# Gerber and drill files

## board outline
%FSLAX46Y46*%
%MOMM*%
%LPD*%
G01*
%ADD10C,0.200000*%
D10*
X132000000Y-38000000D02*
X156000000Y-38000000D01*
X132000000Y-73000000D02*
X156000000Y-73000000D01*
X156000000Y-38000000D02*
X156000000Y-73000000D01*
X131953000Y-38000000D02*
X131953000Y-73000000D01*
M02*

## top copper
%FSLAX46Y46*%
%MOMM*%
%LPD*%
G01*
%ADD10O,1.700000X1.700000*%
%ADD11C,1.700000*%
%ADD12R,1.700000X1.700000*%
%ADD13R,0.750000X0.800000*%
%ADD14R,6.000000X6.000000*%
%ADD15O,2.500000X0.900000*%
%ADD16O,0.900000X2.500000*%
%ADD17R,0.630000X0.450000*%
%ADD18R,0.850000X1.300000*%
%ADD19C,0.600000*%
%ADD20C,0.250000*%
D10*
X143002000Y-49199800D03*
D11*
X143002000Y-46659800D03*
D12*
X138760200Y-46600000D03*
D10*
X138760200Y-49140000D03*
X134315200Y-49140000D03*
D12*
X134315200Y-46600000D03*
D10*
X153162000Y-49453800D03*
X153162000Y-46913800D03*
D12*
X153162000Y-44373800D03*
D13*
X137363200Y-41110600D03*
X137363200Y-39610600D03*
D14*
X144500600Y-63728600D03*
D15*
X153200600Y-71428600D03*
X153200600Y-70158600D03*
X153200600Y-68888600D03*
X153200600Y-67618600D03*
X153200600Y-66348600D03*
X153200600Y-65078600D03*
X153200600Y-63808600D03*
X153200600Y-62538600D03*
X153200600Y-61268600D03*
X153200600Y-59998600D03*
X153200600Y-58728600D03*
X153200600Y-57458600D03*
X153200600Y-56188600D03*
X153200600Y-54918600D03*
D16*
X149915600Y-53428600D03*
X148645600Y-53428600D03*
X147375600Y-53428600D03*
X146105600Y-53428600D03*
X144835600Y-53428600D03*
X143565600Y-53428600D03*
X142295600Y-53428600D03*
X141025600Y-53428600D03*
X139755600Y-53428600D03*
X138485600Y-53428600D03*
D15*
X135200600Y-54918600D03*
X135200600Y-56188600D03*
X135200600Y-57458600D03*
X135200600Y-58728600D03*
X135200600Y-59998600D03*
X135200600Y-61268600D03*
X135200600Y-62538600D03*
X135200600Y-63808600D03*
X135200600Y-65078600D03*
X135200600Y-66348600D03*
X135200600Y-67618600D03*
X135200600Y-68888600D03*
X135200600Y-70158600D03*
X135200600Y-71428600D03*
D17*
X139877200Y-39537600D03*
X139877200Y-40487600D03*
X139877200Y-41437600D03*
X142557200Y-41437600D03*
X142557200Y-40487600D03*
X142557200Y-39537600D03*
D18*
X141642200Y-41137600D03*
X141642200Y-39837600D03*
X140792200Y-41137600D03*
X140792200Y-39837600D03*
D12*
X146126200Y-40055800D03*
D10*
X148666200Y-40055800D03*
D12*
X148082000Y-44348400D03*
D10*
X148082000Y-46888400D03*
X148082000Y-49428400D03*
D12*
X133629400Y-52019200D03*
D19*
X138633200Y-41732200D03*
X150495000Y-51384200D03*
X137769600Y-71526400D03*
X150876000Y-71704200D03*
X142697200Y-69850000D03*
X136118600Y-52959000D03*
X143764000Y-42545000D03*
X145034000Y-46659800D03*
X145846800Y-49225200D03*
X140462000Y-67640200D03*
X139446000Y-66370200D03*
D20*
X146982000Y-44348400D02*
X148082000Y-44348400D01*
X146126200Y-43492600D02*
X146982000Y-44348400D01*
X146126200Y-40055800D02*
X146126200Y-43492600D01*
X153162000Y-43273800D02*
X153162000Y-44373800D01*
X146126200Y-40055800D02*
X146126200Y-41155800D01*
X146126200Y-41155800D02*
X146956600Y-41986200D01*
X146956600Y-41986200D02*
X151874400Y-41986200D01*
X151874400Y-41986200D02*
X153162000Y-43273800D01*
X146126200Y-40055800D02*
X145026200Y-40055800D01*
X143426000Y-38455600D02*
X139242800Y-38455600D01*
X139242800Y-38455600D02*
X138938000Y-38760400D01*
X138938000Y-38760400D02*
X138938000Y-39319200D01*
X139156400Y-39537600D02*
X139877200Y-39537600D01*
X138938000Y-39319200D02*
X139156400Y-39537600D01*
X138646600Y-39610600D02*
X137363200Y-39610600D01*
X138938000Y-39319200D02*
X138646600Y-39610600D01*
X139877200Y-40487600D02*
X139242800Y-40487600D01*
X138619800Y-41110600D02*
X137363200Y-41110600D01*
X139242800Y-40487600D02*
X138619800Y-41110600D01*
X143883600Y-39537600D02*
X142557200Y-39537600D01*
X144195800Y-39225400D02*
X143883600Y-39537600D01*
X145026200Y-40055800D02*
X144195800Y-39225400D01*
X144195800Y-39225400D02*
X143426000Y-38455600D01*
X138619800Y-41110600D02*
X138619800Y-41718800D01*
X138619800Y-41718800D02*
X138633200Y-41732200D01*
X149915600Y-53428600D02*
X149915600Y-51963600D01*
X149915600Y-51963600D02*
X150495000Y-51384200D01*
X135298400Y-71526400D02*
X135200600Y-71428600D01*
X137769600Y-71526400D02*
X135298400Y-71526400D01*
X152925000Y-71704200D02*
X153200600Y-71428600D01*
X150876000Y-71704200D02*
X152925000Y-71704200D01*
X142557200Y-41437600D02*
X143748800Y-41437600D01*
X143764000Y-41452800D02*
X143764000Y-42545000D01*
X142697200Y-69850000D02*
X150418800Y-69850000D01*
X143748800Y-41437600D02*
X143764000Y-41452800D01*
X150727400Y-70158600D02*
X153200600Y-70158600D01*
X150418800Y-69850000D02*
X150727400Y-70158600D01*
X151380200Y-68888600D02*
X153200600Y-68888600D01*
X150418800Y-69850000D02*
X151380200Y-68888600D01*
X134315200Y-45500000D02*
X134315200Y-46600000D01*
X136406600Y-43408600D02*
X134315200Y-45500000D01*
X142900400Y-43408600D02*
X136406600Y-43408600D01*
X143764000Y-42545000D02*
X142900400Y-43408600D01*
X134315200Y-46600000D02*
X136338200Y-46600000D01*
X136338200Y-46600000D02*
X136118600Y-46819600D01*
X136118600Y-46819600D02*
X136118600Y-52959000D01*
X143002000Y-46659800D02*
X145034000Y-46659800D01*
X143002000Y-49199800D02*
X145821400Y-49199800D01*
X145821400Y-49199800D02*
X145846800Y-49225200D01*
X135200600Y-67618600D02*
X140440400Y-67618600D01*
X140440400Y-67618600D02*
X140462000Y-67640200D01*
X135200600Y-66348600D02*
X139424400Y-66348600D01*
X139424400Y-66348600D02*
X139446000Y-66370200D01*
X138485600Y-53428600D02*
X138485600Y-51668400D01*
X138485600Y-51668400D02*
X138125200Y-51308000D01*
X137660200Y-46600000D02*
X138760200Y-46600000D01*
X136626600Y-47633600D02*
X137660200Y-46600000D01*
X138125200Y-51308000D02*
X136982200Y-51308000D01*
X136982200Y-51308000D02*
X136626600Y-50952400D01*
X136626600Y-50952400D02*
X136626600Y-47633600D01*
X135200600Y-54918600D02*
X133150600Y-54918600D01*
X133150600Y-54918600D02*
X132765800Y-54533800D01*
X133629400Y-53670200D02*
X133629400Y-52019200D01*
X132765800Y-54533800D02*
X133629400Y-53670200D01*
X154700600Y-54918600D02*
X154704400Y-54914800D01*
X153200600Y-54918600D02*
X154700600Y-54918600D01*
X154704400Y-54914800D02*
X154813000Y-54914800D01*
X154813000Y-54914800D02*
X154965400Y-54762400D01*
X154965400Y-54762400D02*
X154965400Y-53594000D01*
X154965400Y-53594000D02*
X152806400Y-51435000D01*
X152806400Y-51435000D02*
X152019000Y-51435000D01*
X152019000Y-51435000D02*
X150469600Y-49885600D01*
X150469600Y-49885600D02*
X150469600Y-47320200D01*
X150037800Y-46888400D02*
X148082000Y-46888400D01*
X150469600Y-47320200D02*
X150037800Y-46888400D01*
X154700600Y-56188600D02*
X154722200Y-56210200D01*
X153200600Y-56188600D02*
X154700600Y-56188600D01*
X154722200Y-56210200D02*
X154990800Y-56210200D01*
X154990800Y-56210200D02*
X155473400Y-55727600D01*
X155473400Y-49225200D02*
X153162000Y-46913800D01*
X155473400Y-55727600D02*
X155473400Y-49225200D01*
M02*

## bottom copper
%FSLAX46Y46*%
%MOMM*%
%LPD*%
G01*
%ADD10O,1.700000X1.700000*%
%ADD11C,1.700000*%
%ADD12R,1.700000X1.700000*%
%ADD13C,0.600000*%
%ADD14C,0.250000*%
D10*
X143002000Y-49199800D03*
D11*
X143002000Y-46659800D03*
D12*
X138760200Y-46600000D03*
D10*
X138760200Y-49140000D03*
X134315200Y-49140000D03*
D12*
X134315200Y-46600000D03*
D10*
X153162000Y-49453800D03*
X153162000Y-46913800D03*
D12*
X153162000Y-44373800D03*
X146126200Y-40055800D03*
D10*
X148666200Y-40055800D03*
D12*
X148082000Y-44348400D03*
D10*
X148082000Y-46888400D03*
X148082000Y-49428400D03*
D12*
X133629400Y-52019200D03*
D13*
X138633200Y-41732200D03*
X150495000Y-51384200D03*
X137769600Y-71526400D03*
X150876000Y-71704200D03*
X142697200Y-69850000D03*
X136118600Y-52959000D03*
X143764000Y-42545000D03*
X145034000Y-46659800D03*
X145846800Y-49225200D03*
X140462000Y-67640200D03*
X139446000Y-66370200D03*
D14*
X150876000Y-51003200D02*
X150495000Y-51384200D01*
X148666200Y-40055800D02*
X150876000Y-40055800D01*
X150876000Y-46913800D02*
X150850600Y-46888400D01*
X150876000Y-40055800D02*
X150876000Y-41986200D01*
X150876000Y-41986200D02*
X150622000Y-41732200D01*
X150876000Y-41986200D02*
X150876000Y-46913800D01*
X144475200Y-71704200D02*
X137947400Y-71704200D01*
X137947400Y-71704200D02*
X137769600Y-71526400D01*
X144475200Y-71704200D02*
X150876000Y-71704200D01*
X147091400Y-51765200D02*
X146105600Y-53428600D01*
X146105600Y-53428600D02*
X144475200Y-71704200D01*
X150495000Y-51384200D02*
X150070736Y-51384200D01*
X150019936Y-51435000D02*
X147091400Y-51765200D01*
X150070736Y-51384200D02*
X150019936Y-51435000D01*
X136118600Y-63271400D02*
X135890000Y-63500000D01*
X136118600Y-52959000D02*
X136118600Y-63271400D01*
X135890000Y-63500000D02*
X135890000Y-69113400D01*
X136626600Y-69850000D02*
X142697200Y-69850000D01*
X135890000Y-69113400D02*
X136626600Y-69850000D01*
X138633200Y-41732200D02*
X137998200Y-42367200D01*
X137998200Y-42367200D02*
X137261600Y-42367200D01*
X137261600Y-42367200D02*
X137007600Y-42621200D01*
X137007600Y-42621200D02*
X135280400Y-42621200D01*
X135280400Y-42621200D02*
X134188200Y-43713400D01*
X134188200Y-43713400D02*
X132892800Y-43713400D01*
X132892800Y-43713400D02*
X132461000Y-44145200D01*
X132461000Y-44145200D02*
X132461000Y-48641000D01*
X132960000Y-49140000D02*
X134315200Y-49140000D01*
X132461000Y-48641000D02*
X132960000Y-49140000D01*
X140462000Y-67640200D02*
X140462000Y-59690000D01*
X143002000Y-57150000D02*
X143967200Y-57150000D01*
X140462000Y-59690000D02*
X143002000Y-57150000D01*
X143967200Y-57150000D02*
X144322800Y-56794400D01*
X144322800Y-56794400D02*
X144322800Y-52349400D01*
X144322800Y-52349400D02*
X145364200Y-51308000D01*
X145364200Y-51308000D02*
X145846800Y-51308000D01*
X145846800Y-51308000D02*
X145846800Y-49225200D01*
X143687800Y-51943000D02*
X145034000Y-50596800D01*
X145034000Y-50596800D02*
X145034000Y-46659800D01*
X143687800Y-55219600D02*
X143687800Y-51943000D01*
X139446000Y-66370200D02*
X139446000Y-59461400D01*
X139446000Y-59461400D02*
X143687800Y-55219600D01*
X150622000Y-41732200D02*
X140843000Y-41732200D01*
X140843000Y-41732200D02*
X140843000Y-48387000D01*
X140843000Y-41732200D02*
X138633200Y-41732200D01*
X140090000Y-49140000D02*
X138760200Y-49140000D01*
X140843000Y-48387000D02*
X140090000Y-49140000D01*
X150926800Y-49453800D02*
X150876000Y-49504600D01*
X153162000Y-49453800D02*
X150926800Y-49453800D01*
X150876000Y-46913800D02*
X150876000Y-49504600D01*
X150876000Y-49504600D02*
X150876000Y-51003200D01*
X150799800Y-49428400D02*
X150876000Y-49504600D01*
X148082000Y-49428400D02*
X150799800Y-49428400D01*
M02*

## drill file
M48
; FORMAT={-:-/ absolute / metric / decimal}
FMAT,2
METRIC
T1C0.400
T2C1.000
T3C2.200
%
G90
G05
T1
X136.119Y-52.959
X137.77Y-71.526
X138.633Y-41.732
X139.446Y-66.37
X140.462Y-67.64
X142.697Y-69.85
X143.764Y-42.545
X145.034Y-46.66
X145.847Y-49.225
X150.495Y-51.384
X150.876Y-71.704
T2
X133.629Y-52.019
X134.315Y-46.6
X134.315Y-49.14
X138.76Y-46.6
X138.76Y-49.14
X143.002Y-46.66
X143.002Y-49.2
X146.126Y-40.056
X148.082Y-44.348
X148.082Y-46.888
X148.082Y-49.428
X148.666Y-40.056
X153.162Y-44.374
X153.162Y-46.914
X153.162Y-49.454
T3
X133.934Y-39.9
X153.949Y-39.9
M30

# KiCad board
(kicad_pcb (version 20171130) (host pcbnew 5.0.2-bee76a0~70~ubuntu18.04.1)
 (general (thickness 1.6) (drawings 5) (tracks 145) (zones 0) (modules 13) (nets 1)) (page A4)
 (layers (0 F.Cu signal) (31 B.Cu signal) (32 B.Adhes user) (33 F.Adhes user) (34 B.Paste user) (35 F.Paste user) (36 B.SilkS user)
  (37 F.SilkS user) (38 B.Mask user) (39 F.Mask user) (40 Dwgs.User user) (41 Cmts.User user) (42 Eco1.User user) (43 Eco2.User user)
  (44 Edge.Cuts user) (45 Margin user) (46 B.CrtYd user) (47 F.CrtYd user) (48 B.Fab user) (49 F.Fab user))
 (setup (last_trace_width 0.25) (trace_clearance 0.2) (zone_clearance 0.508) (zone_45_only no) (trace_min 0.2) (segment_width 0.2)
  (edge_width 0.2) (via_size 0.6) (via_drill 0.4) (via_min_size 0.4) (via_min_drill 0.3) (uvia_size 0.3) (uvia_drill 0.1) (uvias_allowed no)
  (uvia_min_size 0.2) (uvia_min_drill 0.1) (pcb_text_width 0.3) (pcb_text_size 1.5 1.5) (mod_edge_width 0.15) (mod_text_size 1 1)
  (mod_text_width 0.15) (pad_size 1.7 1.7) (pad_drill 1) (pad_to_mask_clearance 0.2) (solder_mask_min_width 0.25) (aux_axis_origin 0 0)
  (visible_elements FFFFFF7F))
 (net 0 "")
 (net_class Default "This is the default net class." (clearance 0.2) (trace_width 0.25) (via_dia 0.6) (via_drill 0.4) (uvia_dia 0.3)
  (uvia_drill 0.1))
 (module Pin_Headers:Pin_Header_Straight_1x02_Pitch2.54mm (layer F.Cu) (at 143.002 46.6598)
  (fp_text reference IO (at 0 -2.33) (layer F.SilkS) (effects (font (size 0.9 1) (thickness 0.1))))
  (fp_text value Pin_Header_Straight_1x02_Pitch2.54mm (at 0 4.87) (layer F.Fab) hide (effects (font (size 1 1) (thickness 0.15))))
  (pad 2 thru_hole oval (at 0 2.54) (size 1.7 1.7) (drill 1) (layers *.Cu *.Mask))
  (pad 1 thru_hole circle (at 0 0) (size 1.7 1.7) (drill 1) (layers *.Cu *.Mask)))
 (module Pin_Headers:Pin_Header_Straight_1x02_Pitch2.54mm (layer F.Cu) (at 138.7602 46.6)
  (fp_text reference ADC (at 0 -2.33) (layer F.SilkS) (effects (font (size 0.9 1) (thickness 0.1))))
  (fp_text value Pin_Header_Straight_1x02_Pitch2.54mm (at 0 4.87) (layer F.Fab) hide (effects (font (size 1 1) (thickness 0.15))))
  (pad 1 thru_hole rect (at 0 0) (size 1.7 1.7) (drill 1) (layers *.Cu *.Mask))
  (pad 2 thru_hole oval (at 0 2.54) (size 1.7 1.7) (drill 1) (layers *.Cu *.Mask)))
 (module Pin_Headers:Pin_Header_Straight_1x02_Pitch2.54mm (layer F.Cu) (at 134.3152 46.6)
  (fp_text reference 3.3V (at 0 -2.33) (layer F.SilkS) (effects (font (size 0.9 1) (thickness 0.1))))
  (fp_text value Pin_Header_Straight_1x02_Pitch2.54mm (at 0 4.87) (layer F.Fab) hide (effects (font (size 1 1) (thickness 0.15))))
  (pad 2 thru_hole oval (at 0 2.54) (size 1.7 1.7) (drill 1) (layers *.Cu *.Mask))
  (pad 1 thru_hole rect (at 0 0) (size 1.7 1.7) (drill 1) (layers *.Cu *.Mask)))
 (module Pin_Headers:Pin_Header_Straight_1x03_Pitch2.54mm (layer F.Cu) (at 153.162 44.3738)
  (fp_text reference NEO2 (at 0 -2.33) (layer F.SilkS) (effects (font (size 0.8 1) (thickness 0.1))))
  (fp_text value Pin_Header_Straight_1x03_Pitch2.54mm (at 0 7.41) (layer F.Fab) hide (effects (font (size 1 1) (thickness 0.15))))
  (pad 3 thru_hole oval (at 0 5.08) (size 1.7 1.7) (drill 1) (layers *.Cu *.Mask))
  (pad 2 thru_hole oval (at 0 2.54) (size 1.7 1.7) (drill 1) (layers *.Cu *.Mask))
  (pad 1 thru_hole rect (at 0 0) (size 1.7 1.7) (drill 1) (layers *.Cu *.Mask)))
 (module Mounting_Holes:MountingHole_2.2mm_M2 (layer F.Cu) (at 133.9342 39.9)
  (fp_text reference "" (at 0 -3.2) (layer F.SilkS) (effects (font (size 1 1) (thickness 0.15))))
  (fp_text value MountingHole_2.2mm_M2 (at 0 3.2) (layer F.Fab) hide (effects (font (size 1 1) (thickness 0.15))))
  (pad 1 np_thru_hole circle (at 0 0) (size 2.2 2.2) (drill 2.2) (layers *.Cu *.Mask F.SilkS)))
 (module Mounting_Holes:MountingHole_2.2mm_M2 (layer F.Cu) (at 153.9494 39.9)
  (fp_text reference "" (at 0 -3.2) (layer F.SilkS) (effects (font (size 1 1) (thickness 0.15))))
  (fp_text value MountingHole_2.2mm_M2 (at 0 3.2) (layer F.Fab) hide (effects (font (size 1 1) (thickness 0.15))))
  (pad 1 np_thru_hole circle (at 0 0) (size 2.2 2.2) (drill 2.2) (layers *.Cu *.Mask F.SilkS)))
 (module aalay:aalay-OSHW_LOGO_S (layer B.Cu) (at 139.9794 40.4876)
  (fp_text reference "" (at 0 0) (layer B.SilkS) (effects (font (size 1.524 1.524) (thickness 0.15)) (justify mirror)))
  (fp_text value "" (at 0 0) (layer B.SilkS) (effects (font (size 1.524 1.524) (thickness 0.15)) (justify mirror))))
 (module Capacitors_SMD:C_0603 (layer F.Cu) (at 137.3632 40.3606 90)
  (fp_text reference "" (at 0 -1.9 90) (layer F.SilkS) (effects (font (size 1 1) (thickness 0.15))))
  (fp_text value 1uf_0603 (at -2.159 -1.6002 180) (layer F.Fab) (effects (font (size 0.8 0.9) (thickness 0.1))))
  (pad 1 smd rect (at -0.75 0 90) (size 0.8 0.75) (layers F.Cu F.Paste F.Mask))
  (pad 2 smd rect (at 0.75 0 90) (size 0.8 0.75) (layers F.Cu F.Paste F.Mask)))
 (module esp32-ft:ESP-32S (layer F.Cu) (at 144.148034 61.911262 180)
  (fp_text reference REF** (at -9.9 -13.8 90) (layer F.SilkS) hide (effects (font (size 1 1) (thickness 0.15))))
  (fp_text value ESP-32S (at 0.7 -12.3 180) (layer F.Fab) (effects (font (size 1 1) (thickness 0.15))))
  (pad 39 smd rect (at -0.352566 -1.817338) (size 6 6) (layers F.Cu F.Paste F.Mask))
  (pad 1 smd oval (at -9.052566 -9.517338) (size 2.5 0.9) (layers F.Cu F.Paste F.Mask))
  (pad 2 smd oval (at -9.052566 -8.247338) (size 2.5 0.9) (layers F.Cu F.Paste F.Mask))
  (pad 3 smd oval (at -9.052566 -6.977338) (size 2.5 0.9) (layers F.Cu F.Paste F.Mask))
  (pad 4 smd oval (at -9.052566 -5.707338) (size 2.5 0.9) (layers F.Cu F.Paste F.Mask))
  (pad 5 smd oval (at -9.052566 -4.437338) (size 2.5 0.9) (layers F.Cu F.Paste F.Mask))
  (pad 6 smd oval (at -9.052566 -3.167338) (size 2.5 0.9) (layers F.Cu F.Paste F.Mask))
  (pad 7 smd oval (at -9.052566 -1.897338) (size 2.5 0.9) (layers F.Cu F.Paste F.Mask))
  (pad 8 smd oval (at -9.052566 -0.627338) (size 2.5 0.9) (layers F.Cu F.Paste F.Mask))
  (pad 9 smd oval (at -9.052566 0.642662) (size 2.5 0.9) (layers F.Cu F.Paste F.Mask))
  (pad 10 smd oval (at -9.052566 1.912662) (size 2.5 0.9) (layers F.Cu F.Paste F.Mask))
  (pad 11 smd oval (at -9.052566 3.182662) (size 2.5 0.9) (layers F.Cu F.Paste F.Mask))
  (pad 12 smd oval (at -9.052566 4.452662) (size 2.5 0.9) (layers F.Cu F.Paste F.Mask))
  (pad 13 smd oval (at -9.052566 5.722662) (size 2.5 0.9) (layers F.Cu F.Paste F.Mask))
  (pad 14 smd oval (at -9.052566 6.992662) (size 2.5 0.9) (layers F.Cu F.Paste F.Mask))
  (pad 15 smd oval (at -5.767566 8.482662) (size 0.9 2.5) (layers F.Cu F.Paste F.Mask))
  (pad 16 smd oval (at -4.497566 8.482662) (size 0.9 2.5) (layers F.Cu F.Paste F.Mask))
  (pad 17 smd oval (at -3.227566 8.482662) (size 0.9 2.5) (layers F.Cu F.Paste F.Mask))
  (pad 18 smd oval (at -1.957566 8.482662) (size 0.9 2.5) (layers F.Cu F.Paste F.Mask))
  (pad 19 smd oval (at -0.687566 8.482662) (size 0.9 2.5) (layers F.Cu F.Paste F.Mask))
  (pad 20 smd oval (at 0.582434 8.482662) (size 0.9 2.5) (layers F.Cu F.Paste F.Mask))
  (pad 21 smd oval (at 1.852434 8.482662) (size 0.9 2.5) (layers F.Cu F.Paste F.Mask))
  (pad 22 smd oval (at 3.122434 8.482662) (size 0.9 2.5) (layers F.Cu F.Paste F.Mask))
  (pad 23 smd oval (at 4.392434 8.482662) (size 0.9 2.5) (layers F.Cu F.Paste F.Mask))
  (pad 24 smd oval (at 5.662434 8.482662) (size 0.9 2.5) (layers F.Cu F.Paste F.Mask))
  (pad 25 smd oval (at 8.947434 6.992662) (size 2.5 0.9) (layers F.Cu F.Paste F.Mask))
  (pad 26 smd oval (at 8.947434 5.722662) (size 2.5 0.9) (layers F.Cu F.Paste F.Mask))
  (pad 27 smd oval (at 8.947434 4.452662) (size 2.5 0.9) (layers F.Cu F.Paste F.Mask))
  (pad 28 smd oval (at 8.947434 3.182662) (size 2.5 0.9) (layers F.Cu F.Paste F.Mask))
  (pad 29 smd oval (at 8.947434 1.912662) (size 2.5 0.9) (layers F.Cu F.Paste F.Mask))
  (pad 30 smd oval (at 8.947434 0.642662) (size 2.5 0.9) (layers F.Cu F.Paste F.Mask))
  (pad 31 smd oval (at 8.947434 -0.627338) (size 2.5 0.9) (layers F.Cu F.Paste F.Mask))
  (pad 32 smd oval (at 8.947434 -1.897338) (size 2.5 0.9) (layers F.Cu F.Paste F.Mask))
  (pad 33 smd oval (at 8.947434 -3.167338) (size 2.5 0.9) (layers F.Cu F.Paste F.Mask))
  (pad 34 smd oval (at 8.947434 -4.437338) (size 2.5 0.9) (layers F.Cu F.Paste F.Mask))
  (pad 35 smd oval (at 8.947434 -5.707338) (size 2.5 0.9) (layers F.Cu F.Paste F.Mask))
  (pad 36 smd oval (at 8.947434 -6.977338) (size 2.5 0.9) (layers F.Cu F.Paste F.Mask))
  (pad 37 smd oval (at 8.947434 -8.247338) (size 2.5 0.9) (layers F.Cu F.Paste F.Mask))
  (pad 38 smd oval (at 8.947434 -9.517338) (size 2.5 0.9) (layers F.Cu F.Paste F.Mask)))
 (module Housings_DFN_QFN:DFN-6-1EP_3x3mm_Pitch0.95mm (layer F.Cu) (at 141.2172 40.4876)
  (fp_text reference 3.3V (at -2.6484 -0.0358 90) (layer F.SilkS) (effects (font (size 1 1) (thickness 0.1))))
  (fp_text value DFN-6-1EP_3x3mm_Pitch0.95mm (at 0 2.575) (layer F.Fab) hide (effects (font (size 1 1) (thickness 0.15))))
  (pad 1 smd rect (at -1.34 -0.95) (size 0.63 0.45) (layers F.Cu F.Paste F.Mask))
  (pad 2 smd rect (at -1.34 0) (size 0.63 0.45) (layers F.Cu F.Paste F.Mask))
  (pad 3 smd rect (at -1.34 0.95) (size 0.63 0.45) (layers F.Cu F.Paste F.Mask))
  (pad 4 smd rect (at 1.34 0.95) (size 0.63 0.45) (layers F.Cu F.Paste F.Mask))
  (pad 5 smd rect (at 1.34 0) (size 0.63 0.45) (layers F.Cu F.Paste F.Mask))
  (pad 6 smd rect (at 1.34 -0.95) (size 0.63 0.45) (layers F.Cu F.Paste F.Mask))
  (pad 7 smd rect (at 0.425 0.65) (size 0.85 1.3) (layers F.Cu F.Paste F.Mask) (solder_paste_margin_ratio -0.2))
  (pad 7 smd rect (at 0.425 -0.65) (size 0.85 1.3) (layers F.Cu F.Paste F.Mask) (solder_paste_margin_ratio -0.2))
  (pad 7 smd rect (at -0.425 0.65) (size 0.85 1.3) (layers F.Cu F.Paste F.Mask) (solder_paste_margin_ratio -0.2))
  (pad 7 smd rect (at -0.425 -0.65) (size 0.85 1.3) (layers F.Cu F.Paste F.Mask) (solder_paste_margin_ratio -0.2)))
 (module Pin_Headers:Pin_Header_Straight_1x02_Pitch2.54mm (layer F.Cu) (at 146.1262 40.0558 90)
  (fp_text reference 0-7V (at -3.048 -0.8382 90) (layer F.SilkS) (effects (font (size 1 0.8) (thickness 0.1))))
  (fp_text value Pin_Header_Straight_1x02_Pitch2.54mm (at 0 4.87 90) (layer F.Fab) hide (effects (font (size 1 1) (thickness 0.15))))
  (pad 1 thru_hole rect (at 0 0 90) (size 1.7 1.7) (drill 1) (layers *.Cu *.Mask))
  (pad 2 thru_hole oval (at 0 2.54 90) (size 1.7 1.7) (drill 1) (layers *.Cu *.Mask)))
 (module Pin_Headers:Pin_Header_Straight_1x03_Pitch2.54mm (layer F.Cu) (at 148.082 44.3484)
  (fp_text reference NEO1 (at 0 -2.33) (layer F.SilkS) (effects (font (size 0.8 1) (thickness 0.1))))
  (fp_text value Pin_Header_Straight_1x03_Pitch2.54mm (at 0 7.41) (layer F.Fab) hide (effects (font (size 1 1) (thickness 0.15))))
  (pad 1 thru_hole rect (at 0 0) (size 1.7 1.7) (drill 1) (layers *.Cu *.Mask))
  (pad 2 thru_hole oval (at 0 2.54) (size 1.7 1.7) (drill 1) (layers *.Cu *.Mask))
  (pad 3 thru_hole oval (at 0 5.08) (size 1.7 1.7) (drill 1) (layers *.Cu *.Mask)))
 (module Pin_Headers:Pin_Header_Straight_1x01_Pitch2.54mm (layer F.Cu) (at 133.6294 52.0192)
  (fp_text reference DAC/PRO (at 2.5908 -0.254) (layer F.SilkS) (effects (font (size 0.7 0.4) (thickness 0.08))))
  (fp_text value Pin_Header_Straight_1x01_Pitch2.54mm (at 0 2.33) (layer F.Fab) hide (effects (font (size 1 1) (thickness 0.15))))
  (pad 1 thru_hole rect (at 0 0) (size 1.7 1.7) (drill 1) (layers *.Cu *.Mask)))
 (gr_line (start 132 38) (end 156 38) (angle 90) (layer Edge.Cuts) (width 0.2))
 (gr_line (start 132 73) (end 156 73) (angle 90) (layer Edge.Cuts) (width 0.2))
 (gr_line (start 156 38) (end 156 73) (angle 90) (layer Edge.Cuts) (width 0.2))
 (gr_line (start 131.953 38) (end 131.953 73) (angle 90) (layer Edge.Cuts) (width 0.2))
 (segment (start 146.982 44.3484) (end 148.082 44.3484) (width 0.25) (layer F.Cu) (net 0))
 (segment (start 146.1262 43.4926) (end 146.982 44.3484) (width 0.25) (layer F.Cu) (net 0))
 (segment (start 146.1262 40.0558) (end 146.1262 43.4926) (width 0.25) (layer F.Cu) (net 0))
 (segment (start 153.162 43.2738) (end 153.162 44.3738) (width 0.25) (layer F.Cu) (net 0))
 (segment (start 146.1262 40.0558) (end 146.1262 41.1558) (width 0.25) (layer F.Cu) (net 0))
 (segment (start 146.1262 41.1558) (end 146.9566 41.9862) (width 0.25) (layer F.Cu) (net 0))
 (segment (start 146.9566 41.9862) (end 151.8744 41.9862) (width 0.25) (layer F.Cu) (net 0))
 (segment (start 151.8744 41.9862) (end 153.162 43.2738) (width 0.25) (layer F.Cu) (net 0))
 (segment (start 146.1262 40.0558) (end 145.0262 40.0558) (width 0.25) (layer F.Cu) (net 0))
 (segment (start 143.426 38.4556) (end 139.2428 38.4556) (width 0.25) (layer F.Cu) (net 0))
 (segment (start 139.2428 38.4556) (end 138.938 38.7604) (width 0.25) (layer F.Cu) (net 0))
 (segment (start 138.938 38.7604) (end 138.938 39.3192) (width 0.25) (layer F.Cu) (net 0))
 (segment (start 139.1564 39.5376) (end 139.8772 39.5376) (width 0.25) (layer F.Cu) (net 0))
 (segment (start 138.938 39.3192) (end 139.1564 39.5376) (width 0.25) (layer F.Cu) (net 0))
 (segment (start 138.6466 39.6106) (end 137.3632 39.6106) (width 0.25) (layer F.Cu) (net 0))
 (segment (start 138.938 39.3192) (end 138.6466 39.6106) (width 0.25) (layer F.Cu) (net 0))
 (segment (start 139.8772 40.4876) (end 139.2428 40.4876) (width 0.25) (layer F.Cu) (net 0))
 (segment (start 138.6198 41.1106) (end 137.3632 41.1106) (width 0.25) (layer F.Cu) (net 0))
 (segment (start 139.2428 40.4876) (end 138.6198 41.1106) (width 0.25) (layer F.Cu) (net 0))
 (segment (start 143.8836 39.5376) (end 142.5572 39.5376) (width 0.25) (layer F.Cu) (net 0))
 (segment (start 144.1958 39.2254) (end 143.8836 39.5376) (width 0.25) (layer F.Cu) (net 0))
 (segment (start 145.0262 40.0558) (end 144.1958 39.2254) (width 0.25) (layer F.Cu) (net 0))
 (segment (start 144.1958 39.2254) (end 143.426 38.4556) (width 0.25) (layer F.Cu) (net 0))
 (segment (start 138.6198 41.1106) (end 138.6198 41.7188) (width 0.25) (layer F.Cu) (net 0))
 (via (at 138.6332 41.7322) (size 0.6) (drill 0.4) (layers F.Cu B.Cu) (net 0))
 (segment (start 138.6198 41.7188) (end 138.6332 41.7322) (width 0.25) (layer F.Cu) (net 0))
 (via (at 150.495 51.3842) (size 0.6) (drill 0.4) (layers F.Cu B.Cu) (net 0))
 (segment (start 149.9156 53.4286) (end 149.9156 51.9636) (width 0.25) (layer F.Cu) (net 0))
 (segment (start 149.9156 51.9636) (end 150.495 51.3842) (width 0.25) (layer F.Cu) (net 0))
 (segment (start 150.876 51.0032) (end 150.495 51.3842) (width 0.25) (layer B.Cu) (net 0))
 (segment (start 148.6662 40.0558) (end 150.876 40.0558) (width 0.25) (layer B.Cu) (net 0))
 (segment (start 150.876 46.9138) (end 150.8506 46.8884) (width 0.25) (layer B.Cu) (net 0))
 (segment (start 150.876 40.0558) (end 150.876 41.9862) (width 0.25) (layer B.Cu) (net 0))
 (segment (start 150.876 41.9862) (end 150.622 41.7322) (width 0.25) (layer B.Cu) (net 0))
 (segment (start 150.876 41.9862) (end 150.876 46.9138) (width 0.25) (layer B.Cu) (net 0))
 (via (at 137.7696 71.5264) (size 0.6) (drill 0.4) (layers F.Cu B.Cu) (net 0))
 (segment (start 144.4752 71.7042) (end 137.9474 71.7042) (width 0.25) (layer B.Cu) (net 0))
 (segment (start 137.9474 71.7042) (end 137.7696 71.5264) (width 0.25) (layer B.Cu) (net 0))
 (segment (start 135.2984 71.5264) (end 135.2006 71.4286) (width 0.25) (layer F.Cu) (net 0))
 (segment (start 137.7696 71.5264) (end 135.2984 71.5264) (width 0.25) (layer F.Cu) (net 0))
 (via (at 150.876 71.7042) (size 0.6) (drill 0.4) (layers F.Cu B.Cu) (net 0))
 (segment (start 144.4752 71.7042) (end 150.876 71.7042) (width 0.25) (layer B.Cu) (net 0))
 (segment (start 152.925 71.7042) (end 153.2006 71.4286) (width 0.25) (layer F.Cu) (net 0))
 (segment (start 150.876 71.7042) (end 152.925 71.7042) (width 0.25) (layer F.Cu) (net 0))
 (segment (start 142.5572 41.4376) (end 143.7488 41.4376) (width 0.25) (layer F.Cu) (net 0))
 (segment (start 143.764 41.4528) (end 143.764 42.545) (width 0.25) (layer F.Cu) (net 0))
 (segment (start 142.6972 69.85) (end 150.4188 69.85) (width 0.25) (layer F.Cu) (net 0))
 (via (at 142.6972 69.85) (size 0.6) (drill 0.4) (layers F.Cu B.Cu) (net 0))
 (segment (start 143.7488 41.4376) (end 143.764 41.4528) (width 0.25) (layer F.Cu) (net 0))
 (segment (start 150.7274 70.1586) (end 153.2006 70.1586) (width 0.25) (layer F.Cu) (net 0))
 (segment (start 150.4188 69.85) (end 150.7274 70.1586) (width 0.25) (layer F.Cu) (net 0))
 (segment (start 151.3802 68.8886) (end 153.2006 68.8886) (width 0.25) (layer F.Cu) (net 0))
 (segment (start 150.4188 69.85) (end 151.3802 68.8886) (width 0.25) (layer F.Cu) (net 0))
 (segment (start 147.0914 51.7652) (end 146.1056 53.4286) (width 0.25) (layer B.Cu) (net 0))
 (segment (start 146.1056 53.4286) (end 144.4752 71.7042) (width 0.25) (layer B.Cu) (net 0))
 (segment (start 150.495 51.3842) (end 150.070736 51.3842) (width 0.25) (layer B.Cu) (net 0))
 (segment (start 150.019936 51.435) (end 147.0914 51.7652) (width 0.25) (layer B.Cu) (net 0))
 (segment (start 150.070736 51.3842) (end 150.019936 51.435) (width 0.25) (layer B.Cu) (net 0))
 (segment (start 134.3152 45.5) (end 134.3152 46.6) (width 0.25) (layer F.Cu) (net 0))
 (segment (start 136.4066 43.4086) (end 134.3152 45.5) (width 0.25) (layer F.Cu) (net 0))
 (segment (start 142.9004 43.4086) (end 136.4066 43.4086) (width 0.25) (layer F.Cu) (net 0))
 (segment (start 143.764 42.545) (end 142.9004 43.4086) (width 0.25) (layer F.Cu) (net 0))
 (segment (start 134.3152 46.6) (end 136.3382 46.6) (width 0.25) (layer F.Cu) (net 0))
 (segment (start 136.3382 46.6) (end 136.1186 46.8196) (width 0.25) (layer F.Cu) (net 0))
 (via (at 136.1186 52.959) (size 0.6) (drill 0.4) (layers F.Cu B.Cu) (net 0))
 (segment (start 136.1186 46.8196) (end 136.1186 52.959) (width 0.25) (layer F.Cu) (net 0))
 (segment (start 136.1186 63.2714) (end 135.89 63.5) (width 0.25) (layer B.Cu) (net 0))
 (segment (start 136.1186 52.959) (end 136.1186 63.2714) (width 0.25) (layer B.Cu) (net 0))
 (segment (start 135.89 63.5) (end 135.89 69.1134) (width 0.25) (layer B.Cu) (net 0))
 (segment (start 136.6266 69.85) (end 142.6972 69.85) (width 0.25) (layer B.Cu) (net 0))
 (segment (start 135.89 69.1134) (end 136.6266 69.85) (width 0.25) (layer B.Cu) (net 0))
 (via (at 143.764 42.545) (size 0.6) (drill 0.4) (layers F.Cu B.Cu) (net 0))
 (segment (start 138.6332 41.7322) (end 137.9982 42.3672) (width 0.25) (layer B.Cu) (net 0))
 (segment (start 137.9982 42.3672) (end 137.2616 42.3672) (width 0.25) (layer B.Cu) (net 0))
 (segment (start 137.2616 42.3672) (end 137.0076 42.6212) (width 0.25) (layer B.Cu) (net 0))
 (segment (start 137.0076 42.6212) (end 135.2804 42.6212) (width 0.25) (layer B.Cu) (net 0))
 (segment (start 135.2804 42.6212) (end 134.1882 43.7134) (width 0.25) (layer B.Cu) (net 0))
 (segment (start 134.1882 43.7134) (end 132.8928 43.7134) (width 0.25) (layer B.Cu) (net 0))
 (segment (start 132.8928 43.7134) (end 132.461 44.1452) (width 0.25) (layer B.Cu) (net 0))
 (segment (start 132.461 44.1452) (end 132.461 48.641) (width 0.25) (layer B.Cu) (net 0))
 (segment (start 132.96 49.14) (end 134.3152 49.14) (width 0.25) (layer B.Cu) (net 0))
 (segment (start 132.461 48.641) (end 132.96 49.14) (width 0.25) (layer B.Cu) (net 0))
 (via (at 145.034 46.6598) (size 0.6) (drill 0.4) (layers F.Cu B.Cu) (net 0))
 (segment (start 143.002 46.6598) (end 145.034 46.6598) (width 0.25) (layer F.Cu) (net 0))
 (segment (start 143.002 49.1998) (end 145.8214 49.1998) (width 0.25) (layer F.Cu) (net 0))
 (via (at 145.8468 49.2252) (size 0.6) (drill 0.4) (layers F.Cu B.Cu) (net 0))
 (segment (start 145.8214 49.1998) (end 145.8468 49.2252) (width 0.25) (layer F.Cu) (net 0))
 (segment (start 135.2006 67.6186) (end 140.4404 67.6186) (width 0.25) (layer F.Cu) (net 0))
 (via (at 140.462 67.6402) (size 0.6) (drill 0.4) (layers F.Cu B.Cu) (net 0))
 (segment (start 140.4404 67.6186) (end 140.462 67.6402) (width 0.25) (layer F.Cu) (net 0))
 (segment (start 140.462 67.6402) (end 140.462 59.69) (width 0.25) (layer B.Cu) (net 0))
 (segment (start 143.002 57.15) (end 143.9672 57.15) (width 0.25) (layer B.Cu) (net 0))
 (segment (start 140.462 59.69) (end 143.002 57.15) (width 0.25) (layer B.Cu) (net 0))
 (segment (start 143.9672 57.15) (end 144.3228 56.7944) (width 0.25) (layer B.Cu) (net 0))
 (segment (start 144.3228 56.7944) (end 144.3228 52.3494) (width 0.25) (layer B.Cu) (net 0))
 (segment (start 144.3228 52.3494) (end 145.3642 51.308) (width 0.25) (layer B.Cu) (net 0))
 (segment (start 145.3642 51.308) (end 145.8468 51.308) (width 0.25) (layer B.Cu) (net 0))
 (segment (start 145.8468 51.308) (end 145.8468 49.2252) (width 0.25) (layer B.Cu) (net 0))
 (via (at 139.446 66.3702) (size 0.6) (drill 0.4) (layers F.Cu B.Cu) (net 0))
 (segment (start 135.2006 66.3486) (end 139.4244 66.3486) (width 0.25) (layer F.Cu) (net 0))
 (segment (start 139.4244 66.3486) (end 139.446 66.3702) (width 0.25) (layer F.Cu) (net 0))
 (segment (start 143.6878 51.943) (end 145.034 50.5968) (width 0.25) (layer B.Cu) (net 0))
 (segment (start 145.034 50.5968) (end 145.034 46.6598) (width 0.25) (layer B.Cu) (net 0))
 (segment (start 143.6878 55.2196) (end 143.6878 51.943) (width 0.25) (layer B.Cu) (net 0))
 (segment (start 139.446 66.3702) (end 139.446 59.4614) (width 0.25) (layer B.Cu) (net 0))
 (segment (start 139.446 59.4614) (end 143.6878 55.2196) (width 0.25) (layer B.Cu) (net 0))
 (segment (start 138.4856 53.4286) (end 138.4856 51.6684) (width 0.25) (layer F.Cu) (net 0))
 (segment (start 138.4856 51.6684) (end 138.1252 51.308) (width 0.25) (layer F.Cu) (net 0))
 (segment (start 137.6602 46.6) (end 138.7602 46.6) (width 0.25) (layer F.Cu) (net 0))
 (segment (start 136.6266 47.6336) (end 137.6602 46.6) (width 0.25) (layer F.Cu) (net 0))
 (segment (start 138.1252 51.308) (end 136.9822 51.308) (width 0.25) (layer F.Cu) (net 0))
 (segment (start 136.9822 51.308) (end 136.6266 50.9524) (width 0.25) (layer F.Cu) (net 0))
 (segment (start 136.6266 50.9524) (end 136.6266 47.6336) (width 0.25) (layer F.Cu) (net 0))
 (segment (start 150.622 41.7322) (end 140.843 41.7322) (width 0.25) (layer B.Cu) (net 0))
 (segment (start 140.843 41.7322) (end 140.843 48.387) (width 0.25) (layer B.Cu) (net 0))
 (segment (start 140.843 41.7322) (end 138.6332 41.7322) (width 0.25) (layer B.Cu) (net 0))
 (segment (start 140.09 49.14) (end 138.7602 49.14) (width 0.25) (layer B.Cu) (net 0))
 (segment (start 140.843 48.387) (end 140.09 49.14) (width 0.25) (layer B.Cu) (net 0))
 (segment (start 135.2006 54.9186) (end 133.1506 54.9186) (width 0.25) (layer F.Cu) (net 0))
 (segment (start 133.1506 54.9186) (end 132.7658 54.5338) (width 0.25) (layer F.Cu) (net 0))
 (segment (start 133.6294 53.6702) (end 133.6294 52.0192) (width 0.25) (layer F.Cu) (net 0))
 (segment (start 132.7658 54.5338) (end 133.6294 53.6702) (width 0.25) (layer F.Cu) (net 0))
 (segment (start 150.9268 49.4538) (end 150.876 49.5046) (width 0.25) (layer B.Cu) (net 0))
 (segment (start 153.162 49.4538) (end 150.9268 49.4538) (width 0.25) (layer B.Cu) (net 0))
 (segment (start 150.876 46.9138) (end 150.876 49.5046) (width 0.25) (layer B.Cu) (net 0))
 (segment (start 150.876 49.5046) (end 150.876 51.0032) (width 0.25) (layer B.Cu) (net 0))
 (segment (start 150.7998 49.4284) (end 150.876 49.5046) (width 0.25) (layer B.Cu) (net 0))
 (segment (start 148.082 49.4284) (end 150.7998 49.4284) (width 0.25) (layer B.Cu) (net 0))
 (segment (start 154.7006 54.9186) (end 154.7044 54.9148) (width 0.25) (layer F.Cu) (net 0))
 (segment (start 153.2006 54.9186) (end 154.7006 54.9186) (width 0.25) (layer F.Cu) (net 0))
 (segment (start 154.7044 54.9148) (end 154.813 54.9148) (width 0.25) (layer F.Cu) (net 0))
 (segment (start 154.813 54.9148) (end 154.9654 54.7624) (width 0.25) (layer F.Cu) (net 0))
 (segment (start 154.9654 54.7624) (end 154.9654 53.594) (width 0.25) (layer F.Cu) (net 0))
 (segment (start 154.9654 53.594) (end 152.8064 51.435) (width 0.25) (layer F.Cu) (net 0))
 (segment (start 152.8064 51.435) (end 152.019 51.435) (width 0.25) (layer F.Cu) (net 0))
 (segment (start 152.019 51.435) (end 150.4696 49.8856) (width 0.25) (layer F.Cu) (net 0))
 (segment (start 150.4696 49.8856) (end 150.4696 47.3202) (width 0.25) (layer F.Cu) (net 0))
 (segment (start 150.0378 46.8884) (end 148.082 46.8884) (width 0.25) (layer F.Cu) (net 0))
 (segment (start 150.4696 47.3202) (end 150.0378 46.8884) (width 0.25) (layer F.Cu) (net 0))
 (segment (start 154.7006 56.1886) (end 154.7222 56.2102) (width 0.25) (layer F.Cu) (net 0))
 (segment (start 153.2006 56.1886) (end 154.7006 56.1886) (width 0.25) (layer F.Cu) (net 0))
 (segment (start 154.7222 56.2102) (end 154.9908 56.2102) (width 0.25) (layer F.Cu) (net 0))
 (segment (start 154.9908 56.2102) (end 155.4734 55.7276) (width 0.25) (layer F.Cu) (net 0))
 (segment (start 155.4734 49.2252) (end 153.162 46.9138) (width 0.25) (layer F.Cu) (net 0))
 (segment (start 155.4734 55.7276) (end 155.4734 49.2252) (width 0.25) (layer F.Cu) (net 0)))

